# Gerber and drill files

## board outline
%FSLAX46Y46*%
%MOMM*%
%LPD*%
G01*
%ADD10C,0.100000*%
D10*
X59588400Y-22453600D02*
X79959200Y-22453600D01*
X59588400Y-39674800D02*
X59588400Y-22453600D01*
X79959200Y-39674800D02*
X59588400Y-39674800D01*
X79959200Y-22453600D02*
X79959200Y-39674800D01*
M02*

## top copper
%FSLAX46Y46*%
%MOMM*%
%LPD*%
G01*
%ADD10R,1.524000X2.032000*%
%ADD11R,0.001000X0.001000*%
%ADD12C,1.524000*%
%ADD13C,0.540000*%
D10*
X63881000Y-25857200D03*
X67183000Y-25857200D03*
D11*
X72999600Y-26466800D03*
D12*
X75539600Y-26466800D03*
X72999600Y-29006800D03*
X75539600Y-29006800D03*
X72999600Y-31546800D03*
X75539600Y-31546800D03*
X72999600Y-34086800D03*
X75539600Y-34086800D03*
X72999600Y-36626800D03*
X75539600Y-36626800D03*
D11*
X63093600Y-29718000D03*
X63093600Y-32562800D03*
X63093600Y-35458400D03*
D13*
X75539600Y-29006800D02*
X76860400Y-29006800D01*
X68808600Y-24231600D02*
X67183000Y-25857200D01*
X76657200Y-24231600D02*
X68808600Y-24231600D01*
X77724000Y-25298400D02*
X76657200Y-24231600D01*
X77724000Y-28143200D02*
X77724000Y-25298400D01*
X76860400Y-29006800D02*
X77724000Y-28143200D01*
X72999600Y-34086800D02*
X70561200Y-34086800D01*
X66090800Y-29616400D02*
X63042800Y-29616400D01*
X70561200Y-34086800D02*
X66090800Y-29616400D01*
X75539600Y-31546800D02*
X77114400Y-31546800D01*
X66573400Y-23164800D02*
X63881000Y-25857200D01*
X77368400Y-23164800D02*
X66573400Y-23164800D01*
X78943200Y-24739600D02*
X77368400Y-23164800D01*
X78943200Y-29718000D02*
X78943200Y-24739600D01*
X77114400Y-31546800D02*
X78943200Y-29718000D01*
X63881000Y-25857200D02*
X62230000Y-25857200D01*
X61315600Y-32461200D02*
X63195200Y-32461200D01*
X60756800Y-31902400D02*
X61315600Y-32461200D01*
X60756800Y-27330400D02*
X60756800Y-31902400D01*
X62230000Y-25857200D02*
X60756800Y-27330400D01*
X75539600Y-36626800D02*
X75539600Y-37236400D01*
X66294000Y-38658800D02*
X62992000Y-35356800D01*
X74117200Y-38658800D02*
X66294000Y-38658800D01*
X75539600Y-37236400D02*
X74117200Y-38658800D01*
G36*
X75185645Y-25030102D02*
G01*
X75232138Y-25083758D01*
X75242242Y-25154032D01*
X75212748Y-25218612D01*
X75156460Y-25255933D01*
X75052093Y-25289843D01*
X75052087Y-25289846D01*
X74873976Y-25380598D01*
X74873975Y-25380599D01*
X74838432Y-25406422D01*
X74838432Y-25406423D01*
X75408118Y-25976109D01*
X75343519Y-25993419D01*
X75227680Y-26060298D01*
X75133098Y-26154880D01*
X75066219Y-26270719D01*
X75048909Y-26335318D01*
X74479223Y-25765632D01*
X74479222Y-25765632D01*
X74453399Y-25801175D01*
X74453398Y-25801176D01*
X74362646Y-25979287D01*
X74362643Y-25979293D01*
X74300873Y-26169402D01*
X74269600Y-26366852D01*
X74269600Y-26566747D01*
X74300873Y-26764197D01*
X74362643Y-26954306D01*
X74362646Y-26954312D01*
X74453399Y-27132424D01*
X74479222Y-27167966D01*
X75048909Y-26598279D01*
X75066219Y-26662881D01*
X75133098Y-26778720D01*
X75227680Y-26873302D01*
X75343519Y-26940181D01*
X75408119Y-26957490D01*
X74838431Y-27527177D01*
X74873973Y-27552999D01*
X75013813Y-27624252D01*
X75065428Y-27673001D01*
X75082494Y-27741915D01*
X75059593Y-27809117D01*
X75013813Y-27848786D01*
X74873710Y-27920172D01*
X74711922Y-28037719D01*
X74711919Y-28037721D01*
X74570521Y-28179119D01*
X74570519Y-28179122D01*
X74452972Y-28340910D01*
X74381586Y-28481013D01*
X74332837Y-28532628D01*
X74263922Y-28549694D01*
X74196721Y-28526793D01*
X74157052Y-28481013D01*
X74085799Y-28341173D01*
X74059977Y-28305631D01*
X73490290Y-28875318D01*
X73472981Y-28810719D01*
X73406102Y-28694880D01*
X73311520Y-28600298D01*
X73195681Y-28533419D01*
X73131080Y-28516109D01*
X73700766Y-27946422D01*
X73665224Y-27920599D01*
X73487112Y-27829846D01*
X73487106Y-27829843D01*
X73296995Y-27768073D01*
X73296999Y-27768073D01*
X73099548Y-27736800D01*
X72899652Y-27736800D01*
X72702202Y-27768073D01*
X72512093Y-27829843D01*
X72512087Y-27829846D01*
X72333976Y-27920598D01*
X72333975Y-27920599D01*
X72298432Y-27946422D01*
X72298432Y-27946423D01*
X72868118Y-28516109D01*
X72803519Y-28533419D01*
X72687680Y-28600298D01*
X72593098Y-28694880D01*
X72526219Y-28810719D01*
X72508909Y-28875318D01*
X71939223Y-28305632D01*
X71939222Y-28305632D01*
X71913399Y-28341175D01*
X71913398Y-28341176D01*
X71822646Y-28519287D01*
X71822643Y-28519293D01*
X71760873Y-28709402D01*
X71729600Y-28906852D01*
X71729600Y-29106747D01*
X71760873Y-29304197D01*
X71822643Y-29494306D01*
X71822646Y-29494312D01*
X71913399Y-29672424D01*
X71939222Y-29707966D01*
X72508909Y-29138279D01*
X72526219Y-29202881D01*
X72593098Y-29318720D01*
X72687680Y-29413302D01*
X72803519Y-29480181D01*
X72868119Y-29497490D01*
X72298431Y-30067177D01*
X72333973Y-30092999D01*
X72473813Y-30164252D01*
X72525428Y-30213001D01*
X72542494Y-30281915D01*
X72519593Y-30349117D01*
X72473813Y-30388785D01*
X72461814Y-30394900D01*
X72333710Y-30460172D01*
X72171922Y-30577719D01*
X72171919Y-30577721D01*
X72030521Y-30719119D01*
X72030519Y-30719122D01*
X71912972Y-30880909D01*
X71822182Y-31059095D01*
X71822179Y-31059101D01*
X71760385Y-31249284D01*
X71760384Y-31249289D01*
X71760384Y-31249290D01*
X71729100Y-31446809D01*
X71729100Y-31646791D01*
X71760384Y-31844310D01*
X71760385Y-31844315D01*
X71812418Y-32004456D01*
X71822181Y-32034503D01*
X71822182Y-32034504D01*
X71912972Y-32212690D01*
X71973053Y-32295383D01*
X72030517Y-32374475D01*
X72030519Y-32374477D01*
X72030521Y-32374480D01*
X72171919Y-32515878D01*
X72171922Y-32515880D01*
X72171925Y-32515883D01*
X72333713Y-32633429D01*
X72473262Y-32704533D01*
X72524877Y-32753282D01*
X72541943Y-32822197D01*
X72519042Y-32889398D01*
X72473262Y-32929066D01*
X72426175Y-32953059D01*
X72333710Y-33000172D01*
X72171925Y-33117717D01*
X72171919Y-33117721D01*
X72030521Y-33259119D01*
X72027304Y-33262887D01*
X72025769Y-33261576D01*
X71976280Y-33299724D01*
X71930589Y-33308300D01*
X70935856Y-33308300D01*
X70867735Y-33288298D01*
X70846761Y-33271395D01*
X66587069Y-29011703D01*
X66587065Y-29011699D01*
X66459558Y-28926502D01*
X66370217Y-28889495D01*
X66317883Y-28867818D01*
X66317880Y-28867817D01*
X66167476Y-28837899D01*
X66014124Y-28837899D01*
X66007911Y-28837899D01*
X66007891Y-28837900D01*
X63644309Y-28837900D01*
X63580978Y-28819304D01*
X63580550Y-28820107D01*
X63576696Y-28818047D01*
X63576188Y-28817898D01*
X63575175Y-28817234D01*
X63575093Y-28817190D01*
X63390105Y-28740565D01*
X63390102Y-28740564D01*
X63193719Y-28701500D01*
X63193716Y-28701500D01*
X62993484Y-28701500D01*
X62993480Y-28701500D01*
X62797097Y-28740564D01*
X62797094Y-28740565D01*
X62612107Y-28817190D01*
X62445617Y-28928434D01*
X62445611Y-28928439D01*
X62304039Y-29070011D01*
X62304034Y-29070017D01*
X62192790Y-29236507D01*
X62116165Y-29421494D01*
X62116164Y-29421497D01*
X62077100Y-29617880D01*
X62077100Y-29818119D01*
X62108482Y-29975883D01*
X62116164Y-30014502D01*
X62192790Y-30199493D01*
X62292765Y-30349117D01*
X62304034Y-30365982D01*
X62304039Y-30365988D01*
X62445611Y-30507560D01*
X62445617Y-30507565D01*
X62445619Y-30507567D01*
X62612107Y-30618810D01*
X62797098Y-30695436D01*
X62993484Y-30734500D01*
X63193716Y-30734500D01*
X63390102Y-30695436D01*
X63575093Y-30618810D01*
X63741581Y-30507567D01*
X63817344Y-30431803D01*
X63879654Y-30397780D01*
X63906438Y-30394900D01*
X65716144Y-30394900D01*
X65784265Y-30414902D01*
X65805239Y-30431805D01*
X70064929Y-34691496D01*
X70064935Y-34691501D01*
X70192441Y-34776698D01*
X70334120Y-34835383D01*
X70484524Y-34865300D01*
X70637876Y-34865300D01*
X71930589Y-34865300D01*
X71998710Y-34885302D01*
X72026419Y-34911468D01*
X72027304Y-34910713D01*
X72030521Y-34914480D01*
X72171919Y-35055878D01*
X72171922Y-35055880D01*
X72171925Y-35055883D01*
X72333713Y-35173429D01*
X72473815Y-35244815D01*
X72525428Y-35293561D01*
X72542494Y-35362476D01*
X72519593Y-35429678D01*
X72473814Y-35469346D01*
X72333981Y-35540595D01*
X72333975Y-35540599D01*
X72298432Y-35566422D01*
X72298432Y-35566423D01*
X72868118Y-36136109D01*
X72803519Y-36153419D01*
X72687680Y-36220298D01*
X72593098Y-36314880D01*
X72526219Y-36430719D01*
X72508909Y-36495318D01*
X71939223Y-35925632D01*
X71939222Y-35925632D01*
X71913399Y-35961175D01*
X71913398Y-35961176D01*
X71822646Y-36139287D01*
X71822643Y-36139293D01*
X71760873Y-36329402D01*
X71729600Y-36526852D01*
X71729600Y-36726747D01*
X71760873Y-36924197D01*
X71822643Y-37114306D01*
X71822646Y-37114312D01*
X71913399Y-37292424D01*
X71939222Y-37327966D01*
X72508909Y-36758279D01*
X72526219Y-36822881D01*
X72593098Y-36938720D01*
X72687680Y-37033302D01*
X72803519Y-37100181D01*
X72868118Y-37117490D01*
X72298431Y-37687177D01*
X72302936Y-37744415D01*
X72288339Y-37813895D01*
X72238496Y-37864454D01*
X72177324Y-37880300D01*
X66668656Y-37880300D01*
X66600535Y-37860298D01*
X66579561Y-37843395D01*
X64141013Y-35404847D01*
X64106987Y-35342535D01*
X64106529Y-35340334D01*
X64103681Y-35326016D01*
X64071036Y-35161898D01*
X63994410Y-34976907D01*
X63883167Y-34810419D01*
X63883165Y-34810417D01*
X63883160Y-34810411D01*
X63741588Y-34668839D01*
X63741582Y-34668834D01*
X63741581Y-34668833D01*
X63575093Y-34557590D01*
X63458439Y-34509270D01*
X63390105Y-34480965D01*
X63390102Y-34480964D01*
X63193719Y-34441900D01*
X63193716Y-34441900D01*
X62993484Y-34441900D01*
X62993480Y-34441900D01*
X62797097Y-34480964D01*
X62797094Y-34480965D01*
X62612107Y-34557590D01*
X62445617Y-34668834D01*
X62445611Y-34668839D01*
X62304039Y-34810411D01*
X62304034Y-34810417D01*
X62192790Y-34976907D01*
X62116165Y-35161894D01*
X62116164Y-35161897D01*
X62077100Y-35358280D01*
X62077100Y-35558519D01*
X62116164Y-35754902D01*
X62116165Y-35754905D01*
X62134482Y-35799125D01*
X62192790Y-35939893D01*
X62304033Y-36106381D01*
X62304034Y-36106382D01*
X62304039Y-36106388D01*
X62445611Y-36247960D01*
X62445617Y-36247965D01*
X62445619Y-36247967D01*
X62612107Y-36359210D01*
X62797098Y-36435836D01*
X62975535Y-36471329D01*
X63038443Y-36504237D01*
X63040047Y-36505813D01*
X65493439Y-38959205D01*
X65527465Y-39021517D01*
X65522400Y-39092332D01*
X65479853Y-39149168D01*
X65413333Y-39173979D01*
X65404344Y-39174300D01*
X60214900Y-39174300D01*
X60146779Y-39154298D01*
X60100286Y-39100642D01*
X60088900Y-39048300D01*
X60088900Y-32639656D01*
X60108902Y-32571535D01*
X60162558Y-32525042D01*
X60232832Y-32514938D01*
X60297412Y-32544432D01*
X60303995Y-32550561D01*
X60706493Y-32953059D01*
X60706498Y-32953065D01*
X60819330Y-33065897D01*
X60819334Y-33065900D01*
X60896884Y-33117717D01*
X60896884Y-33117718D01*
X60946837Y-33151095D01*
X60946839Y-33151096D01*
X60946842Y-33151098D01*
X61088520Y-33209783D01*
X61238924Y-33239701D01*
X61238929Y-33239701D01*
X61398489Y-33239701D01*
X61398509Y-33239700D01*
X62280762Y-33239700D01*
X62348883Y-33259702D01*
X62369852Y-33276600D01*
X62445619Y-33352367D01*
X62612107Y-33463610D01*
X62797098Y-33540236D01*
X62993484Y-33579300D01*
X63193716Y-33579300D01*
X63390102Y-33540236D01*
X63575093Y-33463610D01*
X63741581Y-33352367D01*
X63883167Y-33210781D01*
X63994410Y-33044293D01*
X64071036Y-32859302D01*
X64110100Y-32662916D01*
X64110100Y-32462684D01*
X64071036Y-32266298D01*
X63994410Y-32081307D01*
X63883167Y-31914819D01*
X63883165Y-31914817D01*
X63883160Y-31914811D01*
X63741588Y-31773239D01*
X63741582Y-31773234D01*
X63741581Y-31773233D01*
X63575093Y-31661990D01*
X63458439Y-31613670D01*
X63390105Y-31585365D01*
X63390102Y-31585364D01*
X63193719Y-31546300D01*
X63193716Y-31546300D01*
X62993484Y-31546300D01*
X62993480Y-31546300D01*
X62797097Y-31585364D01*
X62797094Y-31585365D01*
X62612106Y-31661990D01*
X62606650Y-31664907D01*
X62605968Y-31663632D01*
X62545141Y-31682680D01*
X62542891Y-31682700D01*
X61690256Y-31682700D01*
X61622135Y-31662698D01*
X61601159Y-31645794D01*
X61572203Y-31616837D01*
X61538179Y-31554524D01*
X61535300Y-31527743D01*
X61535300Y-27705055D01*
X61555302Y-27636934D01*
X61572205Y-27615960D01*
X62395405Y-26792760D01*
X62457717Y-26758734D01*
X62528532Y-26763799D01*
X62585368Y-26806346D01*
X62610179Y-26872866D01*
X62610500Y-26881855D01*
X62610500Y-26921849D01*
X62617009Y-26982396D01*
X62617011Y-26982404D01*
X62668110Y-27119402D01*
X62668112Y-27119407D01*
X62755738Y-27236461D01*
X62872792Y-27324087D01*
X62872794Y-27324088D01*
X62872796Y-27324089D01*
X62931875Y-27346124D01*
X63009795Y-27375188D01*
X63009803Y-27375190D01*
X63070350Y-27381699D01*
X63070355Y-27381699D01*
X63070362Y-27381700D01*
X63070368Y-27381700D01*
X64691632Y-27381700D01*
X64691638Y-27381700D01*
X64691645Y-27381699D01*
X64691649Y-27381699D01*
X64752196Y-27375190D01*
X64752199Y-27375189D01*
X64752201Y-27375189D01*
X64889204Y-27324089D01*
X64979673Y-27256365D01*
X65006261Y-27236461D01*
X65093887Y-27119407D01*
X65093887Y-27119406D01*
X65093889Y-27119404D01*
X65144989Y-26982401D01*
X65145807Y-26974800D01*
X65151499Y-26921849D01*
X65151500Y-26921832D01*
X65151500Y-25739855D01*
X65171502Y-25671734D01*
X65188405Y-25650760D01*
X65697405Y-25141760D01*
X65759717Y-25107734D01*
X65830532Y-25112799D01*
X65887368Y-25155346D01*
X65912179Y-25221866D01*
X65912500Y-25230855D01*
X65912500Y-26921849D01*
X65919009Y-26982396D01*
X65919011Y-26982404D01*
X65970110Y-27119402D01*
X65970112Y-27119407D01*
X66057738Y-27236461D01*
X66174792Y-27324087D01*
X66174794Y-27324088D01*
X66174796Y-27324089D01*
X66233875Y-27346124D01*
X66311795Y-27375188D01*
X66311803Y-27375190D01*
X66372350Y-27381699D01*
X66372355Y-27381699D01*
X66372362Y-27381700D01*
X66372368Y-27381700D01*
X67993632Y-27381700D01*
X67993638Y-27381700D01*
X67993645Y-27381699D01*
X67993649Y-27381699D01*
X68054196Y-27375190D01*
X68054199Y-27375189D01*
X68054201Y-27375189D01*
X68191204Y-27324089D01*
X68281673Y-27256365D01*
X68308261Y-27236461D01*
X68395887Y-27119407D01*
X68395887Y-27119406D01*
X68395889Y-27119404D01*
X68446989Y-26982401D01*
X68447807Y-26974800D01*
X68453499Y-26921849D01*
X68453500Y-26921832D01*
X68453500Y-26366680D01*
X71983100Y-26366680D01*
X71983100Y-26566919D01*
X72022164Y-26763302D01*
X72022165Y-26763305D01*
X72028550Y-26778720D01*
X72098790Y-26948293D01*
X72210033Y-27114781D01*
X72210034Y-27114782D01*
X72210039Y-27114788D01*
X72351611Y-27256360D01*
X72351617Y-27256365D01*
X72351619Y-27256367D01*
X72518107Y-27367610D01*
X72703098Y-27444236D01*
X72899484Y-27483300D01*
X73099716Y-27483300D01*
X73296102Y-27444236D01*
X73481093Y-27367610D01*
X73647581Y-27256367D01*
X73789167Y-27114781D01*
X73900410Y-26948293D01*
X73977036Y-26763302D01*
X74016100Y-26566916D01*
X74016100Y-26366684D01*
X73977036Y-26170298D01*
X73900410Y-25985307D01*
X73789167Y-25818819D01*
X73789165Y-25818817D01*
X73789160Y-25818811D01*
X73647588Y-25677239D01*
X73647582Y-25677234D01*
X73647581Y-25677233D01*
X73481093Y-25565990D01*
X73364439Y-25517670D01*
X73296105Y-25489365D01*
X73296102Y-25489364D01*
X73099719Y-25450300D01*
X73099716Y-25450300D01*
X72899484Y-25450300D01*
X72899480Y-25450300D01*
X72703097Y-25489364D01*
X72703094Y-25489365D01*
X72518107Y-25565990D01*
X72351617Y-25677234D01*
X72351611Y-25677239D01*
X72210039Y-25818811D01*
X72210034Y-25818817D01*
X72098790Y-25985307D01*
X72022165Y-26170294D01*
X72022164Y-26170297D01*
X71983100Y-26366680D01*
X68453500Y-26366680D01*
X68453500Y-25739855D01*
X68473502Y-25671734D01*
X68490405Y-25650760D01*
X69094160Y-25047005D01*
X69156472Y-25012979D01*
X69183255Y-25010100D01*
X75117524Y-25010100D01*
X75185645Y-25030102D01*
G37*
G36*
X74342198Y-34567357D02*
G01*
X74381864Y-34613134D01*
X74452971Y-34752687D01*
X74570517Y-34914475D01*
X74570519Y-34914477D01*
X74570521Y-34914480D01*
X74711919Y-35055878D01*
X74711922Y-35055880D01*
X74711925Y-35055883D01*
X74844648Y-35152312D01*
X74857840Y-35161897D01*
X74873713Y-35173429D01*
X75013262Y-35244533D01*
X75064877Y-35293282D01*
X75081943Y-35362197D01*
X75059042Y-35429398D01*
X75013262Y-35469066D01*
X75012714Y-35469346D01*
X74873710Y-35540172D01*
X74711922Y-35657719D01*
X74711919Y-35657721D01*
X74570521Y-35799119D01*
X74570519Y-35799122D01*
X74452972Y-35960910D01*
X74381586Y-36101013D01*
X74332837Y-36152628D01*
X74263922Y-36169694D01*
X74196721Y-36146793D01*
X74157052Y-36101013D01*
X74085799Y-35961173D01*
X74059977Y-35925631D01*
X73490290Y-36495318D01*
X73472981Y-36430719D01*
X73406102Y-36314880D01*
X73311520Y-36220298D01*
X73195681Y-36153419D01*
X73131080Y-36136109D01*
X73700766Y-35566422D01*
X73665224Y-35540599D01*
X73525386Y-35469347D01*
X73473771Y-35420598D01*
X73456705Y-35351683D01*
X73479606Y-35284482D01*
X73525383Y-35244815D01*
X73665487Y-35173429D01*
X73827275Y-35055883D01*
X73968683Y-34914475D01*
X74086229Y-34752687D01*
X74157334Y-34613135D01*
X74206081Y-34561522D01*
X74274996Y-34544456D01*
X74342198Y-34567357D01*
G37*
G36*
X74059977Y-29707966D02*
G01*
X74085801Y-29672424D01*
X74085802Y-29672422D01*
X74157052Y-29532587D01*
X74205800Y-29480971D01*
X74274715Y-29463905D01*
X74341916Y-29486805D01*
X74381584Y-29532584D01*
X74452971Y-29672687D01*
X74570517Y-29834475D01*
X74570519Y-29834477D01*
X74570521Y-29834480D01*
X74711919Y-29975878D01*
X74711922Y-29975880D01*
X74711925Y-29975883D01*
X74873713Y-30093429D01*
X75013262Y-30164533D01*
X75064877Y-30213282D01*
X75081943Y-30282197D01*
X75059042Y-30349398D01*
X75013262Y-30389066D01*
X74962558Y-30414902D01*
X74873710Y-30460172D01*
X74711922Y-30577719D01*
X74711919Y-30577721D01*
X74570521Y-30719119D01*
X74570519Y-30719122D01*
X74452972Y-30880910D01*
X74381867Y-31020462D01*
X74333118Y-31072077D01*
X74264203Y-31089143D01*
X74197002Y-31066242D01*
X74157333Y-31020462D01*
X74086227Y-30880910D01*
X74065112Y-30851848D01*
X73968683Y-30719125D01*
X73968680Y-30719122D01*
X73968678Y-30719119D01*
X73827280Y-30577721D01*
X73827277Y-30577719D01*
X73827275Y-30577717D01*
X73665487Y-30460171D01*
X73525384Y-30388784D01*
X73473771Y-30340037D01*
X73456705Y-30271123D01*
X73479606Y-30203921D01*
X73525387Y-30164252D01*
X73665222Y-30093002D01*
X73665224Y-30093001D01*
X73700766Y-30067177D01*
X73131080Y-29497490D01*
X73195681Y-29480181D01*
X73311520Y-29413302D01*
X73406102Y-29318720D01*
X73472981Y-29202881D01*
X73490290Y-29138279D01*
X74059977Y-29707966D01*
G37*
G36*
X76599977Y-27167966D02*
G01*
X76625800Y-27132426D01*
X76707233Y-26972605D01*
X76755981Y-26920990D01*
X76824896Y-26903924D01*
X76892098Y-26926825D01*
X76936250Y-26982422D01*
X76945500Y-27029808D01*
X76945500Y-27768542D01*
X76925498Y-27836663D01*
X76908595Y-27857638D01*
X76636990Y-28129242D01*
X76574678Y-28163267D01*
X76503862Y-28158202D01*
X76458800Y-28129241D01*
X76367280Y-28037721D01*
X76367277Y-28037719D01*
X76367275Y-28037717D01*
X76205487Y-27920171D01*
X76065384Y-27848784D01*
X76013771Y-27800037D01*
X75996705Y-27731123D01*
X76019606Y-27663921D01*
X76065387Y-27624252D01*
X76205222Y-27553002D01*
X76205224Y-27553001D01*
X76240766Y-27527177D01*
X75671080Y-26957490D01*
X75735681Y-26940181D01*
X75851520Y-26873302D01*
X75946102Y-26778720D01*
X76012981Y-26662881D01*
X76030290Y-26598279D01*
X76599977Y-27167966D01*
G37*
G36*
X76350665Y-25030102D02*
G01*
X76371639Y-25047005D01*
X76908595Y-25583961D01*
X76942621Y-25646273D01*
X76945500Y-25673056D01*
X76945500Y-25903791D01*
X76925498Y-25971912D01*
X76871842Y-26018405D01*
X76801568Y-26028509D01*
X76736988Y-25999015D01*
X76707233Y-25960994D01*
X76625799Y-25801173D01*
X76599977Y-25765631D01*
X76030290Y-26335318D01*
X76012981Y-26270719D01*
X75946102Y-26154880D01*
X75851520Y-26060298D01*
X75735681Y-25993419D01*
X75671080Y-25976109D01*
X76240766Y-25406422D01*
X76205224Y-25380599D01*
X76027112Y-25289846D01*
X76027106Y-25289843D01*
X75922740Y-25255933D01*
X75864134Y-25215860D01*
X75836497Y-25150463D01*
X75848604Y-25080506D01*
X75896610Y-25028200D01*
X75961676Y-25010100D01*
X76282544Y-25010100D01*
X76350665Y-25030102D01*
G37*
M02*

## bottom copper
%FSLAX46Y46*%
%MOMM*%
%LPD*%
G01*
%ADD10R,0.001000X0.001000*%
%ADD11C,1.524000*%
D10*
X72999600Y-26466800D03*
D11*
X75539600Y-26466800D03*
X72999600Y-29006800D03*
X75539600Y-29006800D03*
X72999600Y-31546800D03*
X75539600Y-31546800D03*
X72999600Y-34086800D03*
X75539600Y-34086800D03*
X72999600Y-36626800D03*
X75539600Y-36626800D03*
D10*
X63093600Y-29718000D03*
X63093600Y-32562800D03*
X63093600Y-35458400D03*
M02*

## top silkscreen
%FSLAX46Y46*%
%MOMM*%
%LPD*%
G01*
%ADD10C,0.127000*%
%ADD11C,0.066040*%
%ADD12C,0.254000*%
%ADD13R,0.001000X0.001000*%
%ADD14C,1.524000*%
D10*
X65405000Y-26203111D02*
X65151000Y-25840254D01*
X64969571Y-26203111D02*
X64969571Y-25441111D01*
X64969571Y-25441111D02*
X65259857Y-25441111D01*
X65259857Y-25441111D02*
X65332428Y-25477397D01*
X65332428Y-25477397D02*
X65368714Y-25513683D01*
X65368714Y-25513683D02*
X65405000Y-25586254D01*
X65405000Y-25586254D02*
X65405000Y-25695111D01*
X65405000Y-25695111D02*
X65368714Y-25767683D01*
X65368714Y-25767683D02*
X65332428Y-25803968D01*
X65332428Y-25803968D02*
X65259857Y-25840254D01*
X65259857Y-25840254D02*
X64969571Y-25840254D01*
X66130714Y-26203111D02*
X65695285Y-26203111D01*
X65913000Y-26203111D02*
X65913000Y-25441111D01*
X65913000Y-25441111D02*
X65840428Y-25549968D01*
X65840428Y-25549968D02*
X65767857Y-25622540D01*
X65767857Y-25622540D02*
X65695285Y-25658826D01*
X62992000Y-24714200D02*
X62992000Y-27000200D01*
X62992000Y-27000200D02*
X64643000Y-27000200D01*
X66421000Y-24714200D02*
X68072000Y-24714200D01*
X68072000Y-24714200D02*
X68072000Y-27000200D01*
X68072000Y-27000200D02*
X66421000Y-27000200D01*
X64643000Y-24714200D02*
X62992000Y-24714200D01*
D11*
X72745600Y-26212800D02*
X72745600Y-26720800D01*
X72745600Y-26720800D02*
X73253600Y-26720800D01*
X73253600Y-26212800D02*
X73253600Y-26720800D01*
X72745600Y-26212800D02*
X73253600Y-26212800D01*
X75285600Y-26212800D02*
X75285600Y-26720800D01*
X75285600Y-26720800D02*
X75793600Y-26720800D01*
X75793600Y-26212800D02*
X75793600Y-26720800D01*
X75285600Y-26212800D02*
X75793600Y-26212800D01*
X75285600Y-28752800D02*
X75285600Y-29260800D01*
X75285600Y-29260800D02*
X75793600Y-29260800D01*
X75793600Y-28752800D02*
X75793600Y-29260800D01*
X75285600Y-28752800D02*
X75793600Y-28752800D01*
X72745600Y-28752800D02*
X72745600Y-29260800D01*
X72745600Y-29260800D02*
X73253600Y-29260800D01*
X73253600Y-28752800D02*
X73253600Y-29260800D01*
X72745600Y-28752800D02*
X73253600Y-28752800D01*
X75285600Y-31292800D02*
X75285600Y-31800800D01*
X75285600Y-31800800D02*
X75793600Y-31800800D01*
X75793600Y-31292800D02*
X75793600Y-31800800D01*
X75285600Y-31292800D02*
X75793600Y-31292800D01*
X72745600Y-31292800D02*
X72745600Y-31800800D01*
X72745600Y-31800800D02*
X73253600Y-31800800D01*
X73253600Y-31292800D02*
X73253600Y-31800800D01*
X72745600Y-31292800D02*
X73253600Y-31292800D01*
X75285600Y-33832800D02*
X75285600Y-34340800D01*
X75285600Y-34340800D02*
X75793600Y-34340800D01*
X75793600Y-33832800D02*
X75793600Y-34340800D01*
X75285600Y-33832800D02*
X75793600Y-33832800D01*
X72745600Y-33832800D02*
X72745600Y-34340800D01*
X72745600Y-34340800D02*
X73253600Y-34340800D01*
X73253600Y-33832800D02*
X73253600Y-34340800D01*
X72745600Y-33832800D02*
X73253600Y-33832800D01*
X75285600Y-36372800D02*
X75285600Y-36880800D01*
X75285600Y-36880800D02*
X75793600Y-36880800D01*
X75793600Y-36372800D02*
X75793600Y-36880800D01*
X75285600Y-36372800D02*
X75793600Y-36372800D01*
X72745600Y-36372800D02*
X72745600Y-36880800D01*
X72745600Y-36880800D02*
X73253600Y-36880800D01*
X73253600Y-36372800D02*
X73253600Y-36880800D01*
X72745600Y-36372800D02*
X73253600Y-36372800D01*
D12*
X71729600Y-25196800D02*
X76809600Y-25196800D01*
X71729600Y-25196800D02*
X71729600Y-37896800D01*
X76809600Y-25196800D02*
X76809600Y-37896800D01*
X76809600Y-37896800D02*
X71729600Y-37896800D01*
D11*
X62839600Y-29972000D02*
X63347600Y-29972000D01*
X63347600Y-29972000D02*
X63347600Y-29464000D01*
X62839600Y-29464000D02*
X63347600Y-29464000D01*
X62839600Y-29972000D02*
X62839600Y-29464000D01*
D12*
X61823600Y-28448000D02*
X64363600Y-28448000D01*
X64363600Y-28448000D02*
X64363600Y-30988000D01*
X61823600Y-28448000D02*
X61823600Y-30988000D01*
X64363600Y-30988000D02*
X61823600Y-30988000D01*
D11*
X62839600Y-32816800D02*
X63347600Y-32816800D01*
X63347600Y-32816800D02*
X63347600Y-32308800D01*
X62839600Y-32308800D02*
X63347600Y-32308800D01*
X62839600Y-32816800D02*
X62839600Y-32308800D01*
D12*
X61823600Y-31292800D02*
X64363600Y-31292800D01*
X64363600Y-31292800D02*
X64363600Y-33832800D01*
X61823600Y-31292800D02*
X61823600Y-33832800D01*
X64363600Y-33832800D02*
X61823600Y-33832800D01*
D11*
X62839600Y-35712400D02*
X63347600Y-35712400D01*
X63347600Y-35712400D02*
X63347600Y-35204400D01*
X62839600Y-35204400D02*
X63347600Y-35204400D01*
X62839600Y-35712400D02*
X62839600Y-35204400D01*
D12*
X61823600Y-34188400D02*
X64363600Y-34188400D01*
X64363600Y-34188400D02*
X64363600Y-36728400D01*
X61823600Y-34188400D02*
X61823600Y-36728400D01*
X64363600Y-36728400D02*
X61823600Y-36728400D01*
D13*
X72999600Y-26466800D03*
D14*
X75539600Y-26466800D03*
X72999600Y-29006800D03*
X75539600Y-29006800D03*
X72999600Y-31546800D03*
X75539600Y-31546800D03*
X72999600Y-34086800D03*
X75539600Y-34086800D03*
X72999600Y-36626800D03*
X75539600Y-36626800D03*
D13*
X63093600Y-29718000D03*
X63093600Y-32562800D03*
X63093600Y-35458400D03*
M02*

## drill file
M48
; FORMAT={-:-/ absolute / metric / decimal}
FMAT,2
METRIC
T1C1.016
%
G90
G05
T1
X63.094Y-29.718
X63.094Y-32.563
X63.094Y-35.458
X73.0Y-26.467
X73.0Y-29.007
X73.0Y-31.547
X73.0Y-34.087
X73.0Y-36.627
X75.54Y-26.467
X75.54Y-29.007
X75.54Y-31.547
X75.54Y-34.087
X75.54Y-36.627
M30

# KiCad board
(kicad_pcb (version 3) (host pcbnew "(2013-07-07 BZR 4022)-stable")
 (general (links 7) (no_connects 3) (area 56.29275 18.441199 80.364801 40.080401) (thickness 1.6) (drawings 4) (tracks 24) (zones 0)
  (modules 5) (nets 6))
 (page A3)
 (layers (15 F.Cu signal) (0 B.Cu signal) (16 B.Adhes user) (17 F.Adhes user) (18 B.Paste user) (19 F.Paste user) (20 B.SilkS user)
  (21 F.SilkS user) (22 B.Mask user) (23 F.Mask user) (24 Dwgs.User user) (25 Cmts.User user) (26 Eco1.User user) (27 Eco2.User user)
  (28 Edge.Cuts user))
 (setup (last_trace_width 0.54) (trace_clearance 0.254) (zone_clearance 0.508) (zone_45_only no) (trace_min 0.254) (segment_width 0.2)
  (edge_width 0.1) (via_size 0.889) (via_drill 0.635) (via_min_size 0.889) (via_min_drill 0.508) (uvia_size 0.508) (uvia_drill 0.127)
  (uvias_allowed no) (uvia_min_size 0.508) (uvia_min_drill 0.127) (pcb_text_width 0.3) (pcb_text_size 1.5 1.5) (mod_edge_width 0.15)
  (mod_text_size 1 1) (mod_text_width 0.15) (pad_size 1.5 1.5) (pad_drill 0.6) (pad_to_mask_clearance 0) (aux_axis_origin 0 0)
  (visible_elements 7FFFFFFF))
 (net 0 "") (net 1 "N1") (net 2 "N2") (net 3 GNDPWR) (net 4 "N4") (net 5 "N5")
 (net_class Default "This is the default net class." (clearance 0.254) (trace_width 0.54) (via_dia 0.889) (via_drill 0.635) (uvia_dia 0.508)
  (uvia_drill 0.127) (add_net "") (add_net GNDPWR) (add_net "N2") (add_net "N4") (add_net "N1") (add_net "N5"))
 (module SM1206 (layer F.Cu) (at 65.532 25.8572)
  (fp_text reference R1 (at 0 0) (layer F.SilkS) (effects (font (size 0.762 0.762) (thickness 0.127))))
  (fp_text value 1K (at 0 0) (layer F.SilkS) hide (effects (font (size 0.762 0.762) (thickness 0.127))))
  (fp_line (start -2.54 -1.143) (end -2.54 1.143) (layer F.SilkS) (width 0.127))
  (fp_line (start -2.54 1.143) (end -0.889 1.143) (layer F.SilkS) (width 0.127))
  (fp_line (start 0.889 -1.143) (end 2.54 -1.143) (layer F.SilkS) (width 0.127))
  (fp_line (start 2.54 -1.143) (end 2.54 1.143) (layer F.SilkS) (width 0.127))
  (fp_line (start 2.54 1.143) (end 0.889 1.143) (layer F.SilkS) (width 0.127))
  (fp_line (start -0.889 -1.143) (end -2.54 -1.143) (layer F.SilkS) (width 0.127))
  (pad 1 smd rect (at -1.651 0) (size 1.524 2.032) (layers F.Cu F.Paste F.Mask) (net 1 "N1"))
  (pad 2 smd rect (at 1.651 0) (size 1.524 2.032) (layers F.Cu F.Paste F.Mask) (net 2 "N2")))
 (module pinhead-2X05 (layer F.Cu) (at 74.2696 31.5468 270)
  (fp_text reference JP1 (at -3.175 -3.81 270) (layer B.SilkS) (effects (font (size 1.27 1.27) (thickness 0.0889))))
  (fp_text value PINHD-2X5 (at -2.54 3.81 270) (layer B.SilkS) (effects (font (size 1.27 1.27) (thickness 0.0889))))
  (fp_line (start -5.334 1.524) (end -4.826 1.524) (layer F.SilkS) (width 0.06604))
  (fp_line (start -4.826 1.524) (end -4.826 1.016) (layer F.SilkS) (width 0.06604))
  (fp_line (start -5.334 1.016) (end -4.826 1.016) (layer F.SilkS) (width 0.06604))
  (fp_line (start -5.334 1.524) (end -5.334 1.016) (layer F.SilkS) (width 0.06604))
  (fp_line (start -5.334 -1.016) (end -4.826 -1.016) (layer F.SilkS) (width 0.06604))
  (fp_line (start -4.826 -1.016) (end -4.826 -1.524) (layer F.SilkS) (width 0.06604))
  (fp_line (start -5.334 -1.524) (end -4.826 -1.524) (layer F.SilkS) (width 0.06604))
  (fp_line (start -5.334 -1.016) (end -5.334 -1.524) (layer F.SilkS) (width 0.06604))
  (fp_line (start -2.794 -1.016) (end -2.286 -1.016) (layer F.SilkS) (width 0.06604))
  (fp_line (start -2.286 -1.016) (end -2.286 -1.524) (layer F.SilkS) (width 0.06604))
  (fp_line (start -2.794 -1.524) (end -2.286 -1.524) (layer F.SilkS) (width 0.06604))
  (fp_line (start -2.794 -1.016) (end -2.794 -1.524) (layer F.SilkS) (width 0.06604))
  (fp_line (start -2.794 1.524) (end -2.286 1.524) (layer F.SilkS) (width 0.06604))
  (fp_line (start -2.286 1.524) (end -2.286 1.016) (layer F.SilkS) (width 0.06604))
  (fp_line (start -2.794 1.016) (end -2.286 1.016) (layer F.SilkS) (width 0.06604))
  (fp_line (start -2.794 1.524) (end -2.794 1.016) (layer F.SilkS) (width 0.06604))
  (fp_line (start -0.254 -1.016) (end 0.254 -1.016) (layer F.SilkS) (width 0.06604))
  (fp_line (start 0.254 -1.016) (end 0.254 -1.524) (layer F.SilkS) (width 0.06604))
  (fp_line (start -0.254 -1.524) (end 0.254 -1.524) (layer F.SilkS) (width 0.06604))
  (fp_line (start -0.254 -1.016) (end -0.254 -1.524) (layer F.SilkS) (width 0.06604))
  (fp_line (start -0.254 1.524) (end 0.254 1.524) (layer F.SilkS) (width 0.06604))
  (fp_line (start 0.254 1.524) (end 0.254 1.016) (layer F.SilkS) (width 0.06604))
  (fp_line (start -0.254 1.016) (end 0.254 1.016) (layer F.SilkS) (width 0.06604))
  (fp_line (start -0.254 1.524) (end -0.254 1.016) (layer F.SilkS) (width 0.06604))
  (fp_line (start 2.286 -1.016) (end 2.794 -1.016) (layer F.SilkS) (width 0.06604))
  (fp_line (start 2.794 -1.016) (end 2.794 -1.524) (layer F.SilkS) (width 0.06604))
  (fp_line (start 2.286 -1.524) (end 2.794 -1.524) (layer F.SilkS) (width 0.06604))
  (fp_line (start 2.286 -1.016) (end 2.286 -1.524) (layer F.SilkS) (width 0.06604))
  (fp_line (start 2.286 1.524) (end 2.794 1.524) (layer F.SilkS) (width 0.06604))
  (fp_line (start 2.794 1.524) (end 2.794 1.016) (layer F.SilkS) (width 0.06604))
  (fp_line (start 2.286 1.016) (end 2.794 1.016) (layer F.SilkS) (width 0.06604))
  (fp_line (start 2.286 1.524) (end 2.286 1.016) (layer F.SilkS) (width 0.06604))
  (fp_line (start 4.826 -1.016) (end 5.334 -1.016) (layer F.SilkS) (width 0.06604))
  (fp_line (start 5.334 -1.016) (end 5.334 -1.524) (layer F.SilkS) (width 0.06604))
  (fp_line (start 4.826 -1.524) (end 5.334 -1.524) (layer F.SilkS) (width 0.06604))
  (fp_line (start 4.826 -1.016) (end 4.826 -1.524) (layer F.SilkS) (width 0.06604))
  (fp_line (start 4.826 1.524) (end 5.334 1.524) (layer F.SilkS) (width 0.06604))
  (fp_line (start 5.334 1.524) (end 5.334 1.016) (layer F.SilkS) (width 0.06604))
  (fp_line (start 4.826 1.016) (end 5.334 1.016) (layer F.SilkS) (width 0.06604))
  (fp_line (start 4.826 1.524) (end 4.826 1.016) (layer F.SilkS) (width 0.06604))
  (fp_line (start -6.35 2.54) (end -6.35 -2.54) (layer F.SilkS) (width 0.254))
  (fp_line (start -6.35 2.54) (end 6.35 2.54) (layer F.SilkS) (width 0.254))
  (fp_line (start -6.35 -2.54) (end 6.35 -2.54) (layer F.SilkS) (width 0.254))
  (fp_line (start 6.35 -2.54) (end 6.35 2.54) (layer F.SilkS) (width 0.254))
  (pad 1 thru_hole rect (at -5.08 1.27 270) (size 1.524 0) (drill 1.016) (layers *.Cu F.Paste F.SilkS F.Mask))
  (pad 2 thru_hole circle (at -5.08 -1.27 270) (size 1.524 3.048) (drill 1.016) (layers *.Cu F.Paste F.SilkS F.Mask) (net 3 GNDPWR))
  (pad 3 thru_hole circle (at -2.54 1.27 270) (size 1.524 3.048) (drill 1.016) (layers *.Cu F.Paste F.SilkS F.Mask) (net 3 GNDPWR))
  (pad 4 thru_hole circle (at -2.54 -1.27 270) (size 1.524 3.048) (drill 1.016) (layers *.Cu F.Paste F.SilkS F.Mask) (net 2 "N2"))
  (pad 5 thru_hole circle (at 0 1.27 270) (size 1.524 3.048) (drill 1.016) (layers *.Cu F.Paste F.SilkS F.Mask))
  (pad 6 thru_hole circle (at 0 -1.27 270) (size 1.524 3.048) (drill 1.016) (layers *.Cu F.Paste F.SilkS F.Mask) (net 1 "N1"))
  (pad 7 thru_hole circle (at 2.54 1.27 270) (size 1.524 3.048) (drill 1.016) (layers *.Cu F.Paste F.SilkS F.Mask) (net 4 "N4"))
  (pad 8 thru_hole circle (at 2.54 -1.27 270) (size 1.524 3.048) (drill 1.016) (layers *.Cu F.Paste F.SilkS F.Mask))
  (pad 9 thru_hole circle (at 5.08 1.27 270) (size 1.524 3.048) (drill 1.016) (layers *.Cu F.Paste F.SilkS F.Mask) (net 3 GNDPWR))
  (pad 10 thru_hole circle (at 5.08 -1.27 270) (size 1.524 3.048) (drill 1.016) (layers *.Cu F.Paste F.SilkS F.Mask) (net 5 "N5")))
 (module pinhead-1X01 (layer F.Cu) (at 63.0936 29.718)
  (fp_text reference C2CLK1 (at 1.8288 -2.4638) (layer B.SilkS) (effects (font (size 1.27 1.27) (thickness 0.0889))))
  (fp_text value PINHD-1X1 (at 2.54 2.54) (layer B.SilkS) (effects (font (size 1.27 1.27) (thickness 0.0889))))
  (fp_line (start -0.254 0.254) (end 0.254 0.254) (layer F.SilkS) (width 0.06604))
  (fp_line (start 0.254 0.254) (end 0.254 -0.254) (layer F.SilkS) (width 0.06604))
  (fp_line (start -0.254 -0.254) (end 0.254 -0.254) (layer F.SilkS) (width 0.06604))
  (fp_line (start -0.254 0.254) (end -0.254 -0.254) (layer F.SilkS) (width 0.06604))
  (fp_line (start -1.27 -1.27) (end 1.27 -1.27) (layer F.SilkS) (width 0.254))
  (fp_line (start 1.27 -1.27) (end 1.27 1.27) (layer F.SilkS) (width 0.254))
  (fp_line (start -1.27 -1.27) (end -1.27 1.27) (layer F.SilkS) (width 0.254))
  (fp_line (start 1.27 1.27) (end -1.27 1.27) (layer F.SilkS) (width 0.254))
  (pad 1 thru_hole rect (at 0 0) (size 1.524 0) (drill 1.016) (layers *.Cu F.Paste F.SilkS F.Mask) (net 4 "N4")))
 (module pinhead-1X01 (layer F.Cu) (at 63.0936 32.5628)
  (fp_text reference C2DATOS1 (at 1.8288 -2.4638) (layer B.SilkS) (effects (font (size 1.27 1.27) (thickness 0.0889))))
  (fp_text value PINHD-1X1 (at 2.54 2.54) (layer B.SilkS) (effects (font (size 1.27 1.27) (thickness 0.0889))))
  (fp_line (start -0.254 0.254) (end 0.254 0.254) (layer F.SilkS) (width 0.06604))
  (fp_line (start 0.254 0.254) (end 0.254 -0.254) (layer F.SilkS) (width 0.06604))
  (fp_line (start -0.254 -0.254) (end 0.254 -0.254) (layer F.SilkS) (width 0.06604))
  (fp_line (start -0.254 0.254) (end -0.254 -0.254) (layer F.SilkS) (width 0.06604))
  (fp_line (start -1.27 -1.27) (end 1.27 -1.27) (layer F.SilkS) (width 0.254))
  (fp_line (start 1.27 -1.27) (end 1.27 1.27) (layer F.SilkS) (width 0.254))
  (fp_line (start -1.27 -1.27) (end -1.27 1.27) (layer F.SilkS) (width 0.254))
  (fp_line (start 1.27 1.27) (end -1.27 1.27) (layer F.SilkS) (width 0.254))
  (pad 1 thru_hole rect (at 0 0) (size 1.524 0) (drill 1.016) (layers *.Cu F.Paste F.SilkS F.Mask) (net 1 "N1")))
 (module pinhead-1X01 (layer F.Cu) (at 63.0936 35.4584)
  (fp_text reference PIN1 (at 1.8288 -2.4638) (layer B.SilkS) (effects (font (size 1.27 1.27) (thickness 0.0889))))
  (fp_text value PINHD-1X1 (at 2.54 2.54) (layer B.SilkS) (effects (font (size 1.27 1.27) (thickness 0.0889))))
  (fp_line (start -0.254 0.254) (end 0.254 0.254) (layer F.SilkS) (width 0.06604))
  (fp_line (start 0.254 0.254) (end 0.254 -0.254) (layer F.SilkS) (width 0.06604))
  (fp_line (start -0.254 -0.254) (end 0.254 -0.254) (layer F.SilkS) (width 0.06604))
  (fp_line (start -0.254 0.254) (end -0.254 -0.254) (layer F.SilkS) (width 0.06604))
  (fp_line (start -1.27 -1.27) (end 1.27 -1.27) (layer F.SilkS) (width 0.254))
  (fp_line (start 1.27 -1.27) (end 1.27 1.27) (layer F.SilkS) (width 0.254))
  (fp_line (start -1.27 -1.27) (end -1.27 1.27) (layer F.SilkS) (width 0.254))
  (fp_line (start 1.27 1.27) (end -1.27 1.27) (layer F.SilkS) (width 0.254))
  (pad 1 thru_hole rect (at 0 0) (size 1.524 0) (drill 1.016) (layers *.Cu F.Paste F.SilkS F.Mask) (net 5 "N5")))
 (gr_line (start 59.5884 22.4536) (end 79.9592 22.4536) (angle 90) (layer Edge.Cuts) (width 0.1))
 (gr_line (start 59.5884 39.6748) (end 59.5884 22.4536) (angle 90) (layer Edge.Cuts) (width 0.1))
 (gr_line (start 79.9592 39.6748) (end 59.5884 39.6748) (angle 90) (layer Edge.Cuts) (width 0.1))
 (gr_line (start 79.9592 22.4536) (end 79.9592 39.6748) (angle 90) (layer Edge.Cuts) (width 0.1))
 (segment (start 75.5396 29.0068) (end 76.8604 29.0068) (width 0.54) (layer F.Cu) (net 2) (status 400000))
 (segment (start 68.8086 24.2316) (end 67.183 25.8572) (width 0.54) (layer F.Cu) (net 2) (status 800000))
 (segment (start 76.6572 24.2316) (end 68.8086 24.2316) (width 0.54) (layer F.Cu) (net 2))
 (segment (start 77.724 25.2984) (end 76.6572 24.2316) (width 0.54) (layer F.Cu) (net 2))
 (segment (start 77.724 28.1432) (end 77.724 25.2984) (width 0.54) (layer F.Cu) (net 2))
 (segment (start 76.8604 29.0068) (end 77.724 28.1432) (width 0.54) (layer F.Cu) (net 2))
 (segment (start 72.9996 34.0868) (end 70.5612 34.0868) (width 0.54) (layer F.Cu) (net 4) (status 400000))
 (segment (start 66.0908 29.6164) (end 63.0428 29.6164) (width 0.54) (layer F.Cu) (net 4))
 (segment (start 70.5612 34.0868) (end 66.0908 29.6164) (width 0.54) (layer F.Cu) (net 4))
 (segment (start 75.5396 31.5468) (end 77.1144 31.5468) (width 0.54) (layer F.Cu) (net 1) (status 400000))
 (segment (start 66.5734 23.1648) (end 63.881 25.8572) (width 0.54) (layer F.Cu) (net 1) (status 800000))
 (segment (start 77.3684 23.1648) (end 66.5734 23.1648) (width 0.54) (layer F.Cu) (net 1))
 (segment (start 78.9432 24.7396) (end 77.3684 23.1648) (width 0.54) (layer F.Cu) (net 1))
 (segment (start 78.9432 29.718) (end 78.9432 24.7396) (width 0.54) (layer F.Cu) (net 1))
 (segment (start 77.1144 31.5468) (end 78.9432 29.718) (width 0.54) (layer F.Cu) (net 1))
 (segment (start 63.881 25.8572) (end 62.23 25.8572) (width 0.54) (layer F.Cu) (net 1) (status 400000))
 (segment (start 61.3156 32.4612) (end 63.1952 32.4612) (width 0.54) (layer F.Cu) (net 1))
 (segment (start 60.7568 31.9024) (end 61.3156 32.4612) (width 0.54) (layer F.Cu) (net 1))
 (segment (start 60.7568 27.3304) (end 60.7568 31.9024) (width 0.54) (layer F.Cu) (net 1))
 (segment (start 62.23 25.8572) (end 60.7568 27.3304) (width 0.54) (layer F.Cu) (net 1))
 (segment (start 75.5396 36.6268) (end 75.5396 37.2364) (width 0.54) (layer F.Cu) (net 5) (status C00000))
 (segment (start 66.294 38.6588) (end 62.992 35.3568) (width 0.54) (layer F.Cu) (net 5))
 (segment (start 74.1172 38.6588) (end 66.294 38.6588) (width 0.54) (layer F.Cu) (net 5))
 (segment (start 75.5396 37.2364) (end 74.1172 38.6588) (width 0.54) (layer F.Cu) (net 5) (status 400000))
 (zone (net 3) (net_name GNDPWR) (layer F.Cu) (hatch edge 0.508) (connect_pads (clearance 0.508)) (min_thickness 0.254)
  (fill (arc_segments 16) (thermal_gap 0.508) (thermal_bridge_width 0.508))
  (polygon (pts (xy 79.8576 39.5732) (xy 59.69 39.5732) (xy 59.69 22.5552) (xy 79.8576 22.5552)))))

